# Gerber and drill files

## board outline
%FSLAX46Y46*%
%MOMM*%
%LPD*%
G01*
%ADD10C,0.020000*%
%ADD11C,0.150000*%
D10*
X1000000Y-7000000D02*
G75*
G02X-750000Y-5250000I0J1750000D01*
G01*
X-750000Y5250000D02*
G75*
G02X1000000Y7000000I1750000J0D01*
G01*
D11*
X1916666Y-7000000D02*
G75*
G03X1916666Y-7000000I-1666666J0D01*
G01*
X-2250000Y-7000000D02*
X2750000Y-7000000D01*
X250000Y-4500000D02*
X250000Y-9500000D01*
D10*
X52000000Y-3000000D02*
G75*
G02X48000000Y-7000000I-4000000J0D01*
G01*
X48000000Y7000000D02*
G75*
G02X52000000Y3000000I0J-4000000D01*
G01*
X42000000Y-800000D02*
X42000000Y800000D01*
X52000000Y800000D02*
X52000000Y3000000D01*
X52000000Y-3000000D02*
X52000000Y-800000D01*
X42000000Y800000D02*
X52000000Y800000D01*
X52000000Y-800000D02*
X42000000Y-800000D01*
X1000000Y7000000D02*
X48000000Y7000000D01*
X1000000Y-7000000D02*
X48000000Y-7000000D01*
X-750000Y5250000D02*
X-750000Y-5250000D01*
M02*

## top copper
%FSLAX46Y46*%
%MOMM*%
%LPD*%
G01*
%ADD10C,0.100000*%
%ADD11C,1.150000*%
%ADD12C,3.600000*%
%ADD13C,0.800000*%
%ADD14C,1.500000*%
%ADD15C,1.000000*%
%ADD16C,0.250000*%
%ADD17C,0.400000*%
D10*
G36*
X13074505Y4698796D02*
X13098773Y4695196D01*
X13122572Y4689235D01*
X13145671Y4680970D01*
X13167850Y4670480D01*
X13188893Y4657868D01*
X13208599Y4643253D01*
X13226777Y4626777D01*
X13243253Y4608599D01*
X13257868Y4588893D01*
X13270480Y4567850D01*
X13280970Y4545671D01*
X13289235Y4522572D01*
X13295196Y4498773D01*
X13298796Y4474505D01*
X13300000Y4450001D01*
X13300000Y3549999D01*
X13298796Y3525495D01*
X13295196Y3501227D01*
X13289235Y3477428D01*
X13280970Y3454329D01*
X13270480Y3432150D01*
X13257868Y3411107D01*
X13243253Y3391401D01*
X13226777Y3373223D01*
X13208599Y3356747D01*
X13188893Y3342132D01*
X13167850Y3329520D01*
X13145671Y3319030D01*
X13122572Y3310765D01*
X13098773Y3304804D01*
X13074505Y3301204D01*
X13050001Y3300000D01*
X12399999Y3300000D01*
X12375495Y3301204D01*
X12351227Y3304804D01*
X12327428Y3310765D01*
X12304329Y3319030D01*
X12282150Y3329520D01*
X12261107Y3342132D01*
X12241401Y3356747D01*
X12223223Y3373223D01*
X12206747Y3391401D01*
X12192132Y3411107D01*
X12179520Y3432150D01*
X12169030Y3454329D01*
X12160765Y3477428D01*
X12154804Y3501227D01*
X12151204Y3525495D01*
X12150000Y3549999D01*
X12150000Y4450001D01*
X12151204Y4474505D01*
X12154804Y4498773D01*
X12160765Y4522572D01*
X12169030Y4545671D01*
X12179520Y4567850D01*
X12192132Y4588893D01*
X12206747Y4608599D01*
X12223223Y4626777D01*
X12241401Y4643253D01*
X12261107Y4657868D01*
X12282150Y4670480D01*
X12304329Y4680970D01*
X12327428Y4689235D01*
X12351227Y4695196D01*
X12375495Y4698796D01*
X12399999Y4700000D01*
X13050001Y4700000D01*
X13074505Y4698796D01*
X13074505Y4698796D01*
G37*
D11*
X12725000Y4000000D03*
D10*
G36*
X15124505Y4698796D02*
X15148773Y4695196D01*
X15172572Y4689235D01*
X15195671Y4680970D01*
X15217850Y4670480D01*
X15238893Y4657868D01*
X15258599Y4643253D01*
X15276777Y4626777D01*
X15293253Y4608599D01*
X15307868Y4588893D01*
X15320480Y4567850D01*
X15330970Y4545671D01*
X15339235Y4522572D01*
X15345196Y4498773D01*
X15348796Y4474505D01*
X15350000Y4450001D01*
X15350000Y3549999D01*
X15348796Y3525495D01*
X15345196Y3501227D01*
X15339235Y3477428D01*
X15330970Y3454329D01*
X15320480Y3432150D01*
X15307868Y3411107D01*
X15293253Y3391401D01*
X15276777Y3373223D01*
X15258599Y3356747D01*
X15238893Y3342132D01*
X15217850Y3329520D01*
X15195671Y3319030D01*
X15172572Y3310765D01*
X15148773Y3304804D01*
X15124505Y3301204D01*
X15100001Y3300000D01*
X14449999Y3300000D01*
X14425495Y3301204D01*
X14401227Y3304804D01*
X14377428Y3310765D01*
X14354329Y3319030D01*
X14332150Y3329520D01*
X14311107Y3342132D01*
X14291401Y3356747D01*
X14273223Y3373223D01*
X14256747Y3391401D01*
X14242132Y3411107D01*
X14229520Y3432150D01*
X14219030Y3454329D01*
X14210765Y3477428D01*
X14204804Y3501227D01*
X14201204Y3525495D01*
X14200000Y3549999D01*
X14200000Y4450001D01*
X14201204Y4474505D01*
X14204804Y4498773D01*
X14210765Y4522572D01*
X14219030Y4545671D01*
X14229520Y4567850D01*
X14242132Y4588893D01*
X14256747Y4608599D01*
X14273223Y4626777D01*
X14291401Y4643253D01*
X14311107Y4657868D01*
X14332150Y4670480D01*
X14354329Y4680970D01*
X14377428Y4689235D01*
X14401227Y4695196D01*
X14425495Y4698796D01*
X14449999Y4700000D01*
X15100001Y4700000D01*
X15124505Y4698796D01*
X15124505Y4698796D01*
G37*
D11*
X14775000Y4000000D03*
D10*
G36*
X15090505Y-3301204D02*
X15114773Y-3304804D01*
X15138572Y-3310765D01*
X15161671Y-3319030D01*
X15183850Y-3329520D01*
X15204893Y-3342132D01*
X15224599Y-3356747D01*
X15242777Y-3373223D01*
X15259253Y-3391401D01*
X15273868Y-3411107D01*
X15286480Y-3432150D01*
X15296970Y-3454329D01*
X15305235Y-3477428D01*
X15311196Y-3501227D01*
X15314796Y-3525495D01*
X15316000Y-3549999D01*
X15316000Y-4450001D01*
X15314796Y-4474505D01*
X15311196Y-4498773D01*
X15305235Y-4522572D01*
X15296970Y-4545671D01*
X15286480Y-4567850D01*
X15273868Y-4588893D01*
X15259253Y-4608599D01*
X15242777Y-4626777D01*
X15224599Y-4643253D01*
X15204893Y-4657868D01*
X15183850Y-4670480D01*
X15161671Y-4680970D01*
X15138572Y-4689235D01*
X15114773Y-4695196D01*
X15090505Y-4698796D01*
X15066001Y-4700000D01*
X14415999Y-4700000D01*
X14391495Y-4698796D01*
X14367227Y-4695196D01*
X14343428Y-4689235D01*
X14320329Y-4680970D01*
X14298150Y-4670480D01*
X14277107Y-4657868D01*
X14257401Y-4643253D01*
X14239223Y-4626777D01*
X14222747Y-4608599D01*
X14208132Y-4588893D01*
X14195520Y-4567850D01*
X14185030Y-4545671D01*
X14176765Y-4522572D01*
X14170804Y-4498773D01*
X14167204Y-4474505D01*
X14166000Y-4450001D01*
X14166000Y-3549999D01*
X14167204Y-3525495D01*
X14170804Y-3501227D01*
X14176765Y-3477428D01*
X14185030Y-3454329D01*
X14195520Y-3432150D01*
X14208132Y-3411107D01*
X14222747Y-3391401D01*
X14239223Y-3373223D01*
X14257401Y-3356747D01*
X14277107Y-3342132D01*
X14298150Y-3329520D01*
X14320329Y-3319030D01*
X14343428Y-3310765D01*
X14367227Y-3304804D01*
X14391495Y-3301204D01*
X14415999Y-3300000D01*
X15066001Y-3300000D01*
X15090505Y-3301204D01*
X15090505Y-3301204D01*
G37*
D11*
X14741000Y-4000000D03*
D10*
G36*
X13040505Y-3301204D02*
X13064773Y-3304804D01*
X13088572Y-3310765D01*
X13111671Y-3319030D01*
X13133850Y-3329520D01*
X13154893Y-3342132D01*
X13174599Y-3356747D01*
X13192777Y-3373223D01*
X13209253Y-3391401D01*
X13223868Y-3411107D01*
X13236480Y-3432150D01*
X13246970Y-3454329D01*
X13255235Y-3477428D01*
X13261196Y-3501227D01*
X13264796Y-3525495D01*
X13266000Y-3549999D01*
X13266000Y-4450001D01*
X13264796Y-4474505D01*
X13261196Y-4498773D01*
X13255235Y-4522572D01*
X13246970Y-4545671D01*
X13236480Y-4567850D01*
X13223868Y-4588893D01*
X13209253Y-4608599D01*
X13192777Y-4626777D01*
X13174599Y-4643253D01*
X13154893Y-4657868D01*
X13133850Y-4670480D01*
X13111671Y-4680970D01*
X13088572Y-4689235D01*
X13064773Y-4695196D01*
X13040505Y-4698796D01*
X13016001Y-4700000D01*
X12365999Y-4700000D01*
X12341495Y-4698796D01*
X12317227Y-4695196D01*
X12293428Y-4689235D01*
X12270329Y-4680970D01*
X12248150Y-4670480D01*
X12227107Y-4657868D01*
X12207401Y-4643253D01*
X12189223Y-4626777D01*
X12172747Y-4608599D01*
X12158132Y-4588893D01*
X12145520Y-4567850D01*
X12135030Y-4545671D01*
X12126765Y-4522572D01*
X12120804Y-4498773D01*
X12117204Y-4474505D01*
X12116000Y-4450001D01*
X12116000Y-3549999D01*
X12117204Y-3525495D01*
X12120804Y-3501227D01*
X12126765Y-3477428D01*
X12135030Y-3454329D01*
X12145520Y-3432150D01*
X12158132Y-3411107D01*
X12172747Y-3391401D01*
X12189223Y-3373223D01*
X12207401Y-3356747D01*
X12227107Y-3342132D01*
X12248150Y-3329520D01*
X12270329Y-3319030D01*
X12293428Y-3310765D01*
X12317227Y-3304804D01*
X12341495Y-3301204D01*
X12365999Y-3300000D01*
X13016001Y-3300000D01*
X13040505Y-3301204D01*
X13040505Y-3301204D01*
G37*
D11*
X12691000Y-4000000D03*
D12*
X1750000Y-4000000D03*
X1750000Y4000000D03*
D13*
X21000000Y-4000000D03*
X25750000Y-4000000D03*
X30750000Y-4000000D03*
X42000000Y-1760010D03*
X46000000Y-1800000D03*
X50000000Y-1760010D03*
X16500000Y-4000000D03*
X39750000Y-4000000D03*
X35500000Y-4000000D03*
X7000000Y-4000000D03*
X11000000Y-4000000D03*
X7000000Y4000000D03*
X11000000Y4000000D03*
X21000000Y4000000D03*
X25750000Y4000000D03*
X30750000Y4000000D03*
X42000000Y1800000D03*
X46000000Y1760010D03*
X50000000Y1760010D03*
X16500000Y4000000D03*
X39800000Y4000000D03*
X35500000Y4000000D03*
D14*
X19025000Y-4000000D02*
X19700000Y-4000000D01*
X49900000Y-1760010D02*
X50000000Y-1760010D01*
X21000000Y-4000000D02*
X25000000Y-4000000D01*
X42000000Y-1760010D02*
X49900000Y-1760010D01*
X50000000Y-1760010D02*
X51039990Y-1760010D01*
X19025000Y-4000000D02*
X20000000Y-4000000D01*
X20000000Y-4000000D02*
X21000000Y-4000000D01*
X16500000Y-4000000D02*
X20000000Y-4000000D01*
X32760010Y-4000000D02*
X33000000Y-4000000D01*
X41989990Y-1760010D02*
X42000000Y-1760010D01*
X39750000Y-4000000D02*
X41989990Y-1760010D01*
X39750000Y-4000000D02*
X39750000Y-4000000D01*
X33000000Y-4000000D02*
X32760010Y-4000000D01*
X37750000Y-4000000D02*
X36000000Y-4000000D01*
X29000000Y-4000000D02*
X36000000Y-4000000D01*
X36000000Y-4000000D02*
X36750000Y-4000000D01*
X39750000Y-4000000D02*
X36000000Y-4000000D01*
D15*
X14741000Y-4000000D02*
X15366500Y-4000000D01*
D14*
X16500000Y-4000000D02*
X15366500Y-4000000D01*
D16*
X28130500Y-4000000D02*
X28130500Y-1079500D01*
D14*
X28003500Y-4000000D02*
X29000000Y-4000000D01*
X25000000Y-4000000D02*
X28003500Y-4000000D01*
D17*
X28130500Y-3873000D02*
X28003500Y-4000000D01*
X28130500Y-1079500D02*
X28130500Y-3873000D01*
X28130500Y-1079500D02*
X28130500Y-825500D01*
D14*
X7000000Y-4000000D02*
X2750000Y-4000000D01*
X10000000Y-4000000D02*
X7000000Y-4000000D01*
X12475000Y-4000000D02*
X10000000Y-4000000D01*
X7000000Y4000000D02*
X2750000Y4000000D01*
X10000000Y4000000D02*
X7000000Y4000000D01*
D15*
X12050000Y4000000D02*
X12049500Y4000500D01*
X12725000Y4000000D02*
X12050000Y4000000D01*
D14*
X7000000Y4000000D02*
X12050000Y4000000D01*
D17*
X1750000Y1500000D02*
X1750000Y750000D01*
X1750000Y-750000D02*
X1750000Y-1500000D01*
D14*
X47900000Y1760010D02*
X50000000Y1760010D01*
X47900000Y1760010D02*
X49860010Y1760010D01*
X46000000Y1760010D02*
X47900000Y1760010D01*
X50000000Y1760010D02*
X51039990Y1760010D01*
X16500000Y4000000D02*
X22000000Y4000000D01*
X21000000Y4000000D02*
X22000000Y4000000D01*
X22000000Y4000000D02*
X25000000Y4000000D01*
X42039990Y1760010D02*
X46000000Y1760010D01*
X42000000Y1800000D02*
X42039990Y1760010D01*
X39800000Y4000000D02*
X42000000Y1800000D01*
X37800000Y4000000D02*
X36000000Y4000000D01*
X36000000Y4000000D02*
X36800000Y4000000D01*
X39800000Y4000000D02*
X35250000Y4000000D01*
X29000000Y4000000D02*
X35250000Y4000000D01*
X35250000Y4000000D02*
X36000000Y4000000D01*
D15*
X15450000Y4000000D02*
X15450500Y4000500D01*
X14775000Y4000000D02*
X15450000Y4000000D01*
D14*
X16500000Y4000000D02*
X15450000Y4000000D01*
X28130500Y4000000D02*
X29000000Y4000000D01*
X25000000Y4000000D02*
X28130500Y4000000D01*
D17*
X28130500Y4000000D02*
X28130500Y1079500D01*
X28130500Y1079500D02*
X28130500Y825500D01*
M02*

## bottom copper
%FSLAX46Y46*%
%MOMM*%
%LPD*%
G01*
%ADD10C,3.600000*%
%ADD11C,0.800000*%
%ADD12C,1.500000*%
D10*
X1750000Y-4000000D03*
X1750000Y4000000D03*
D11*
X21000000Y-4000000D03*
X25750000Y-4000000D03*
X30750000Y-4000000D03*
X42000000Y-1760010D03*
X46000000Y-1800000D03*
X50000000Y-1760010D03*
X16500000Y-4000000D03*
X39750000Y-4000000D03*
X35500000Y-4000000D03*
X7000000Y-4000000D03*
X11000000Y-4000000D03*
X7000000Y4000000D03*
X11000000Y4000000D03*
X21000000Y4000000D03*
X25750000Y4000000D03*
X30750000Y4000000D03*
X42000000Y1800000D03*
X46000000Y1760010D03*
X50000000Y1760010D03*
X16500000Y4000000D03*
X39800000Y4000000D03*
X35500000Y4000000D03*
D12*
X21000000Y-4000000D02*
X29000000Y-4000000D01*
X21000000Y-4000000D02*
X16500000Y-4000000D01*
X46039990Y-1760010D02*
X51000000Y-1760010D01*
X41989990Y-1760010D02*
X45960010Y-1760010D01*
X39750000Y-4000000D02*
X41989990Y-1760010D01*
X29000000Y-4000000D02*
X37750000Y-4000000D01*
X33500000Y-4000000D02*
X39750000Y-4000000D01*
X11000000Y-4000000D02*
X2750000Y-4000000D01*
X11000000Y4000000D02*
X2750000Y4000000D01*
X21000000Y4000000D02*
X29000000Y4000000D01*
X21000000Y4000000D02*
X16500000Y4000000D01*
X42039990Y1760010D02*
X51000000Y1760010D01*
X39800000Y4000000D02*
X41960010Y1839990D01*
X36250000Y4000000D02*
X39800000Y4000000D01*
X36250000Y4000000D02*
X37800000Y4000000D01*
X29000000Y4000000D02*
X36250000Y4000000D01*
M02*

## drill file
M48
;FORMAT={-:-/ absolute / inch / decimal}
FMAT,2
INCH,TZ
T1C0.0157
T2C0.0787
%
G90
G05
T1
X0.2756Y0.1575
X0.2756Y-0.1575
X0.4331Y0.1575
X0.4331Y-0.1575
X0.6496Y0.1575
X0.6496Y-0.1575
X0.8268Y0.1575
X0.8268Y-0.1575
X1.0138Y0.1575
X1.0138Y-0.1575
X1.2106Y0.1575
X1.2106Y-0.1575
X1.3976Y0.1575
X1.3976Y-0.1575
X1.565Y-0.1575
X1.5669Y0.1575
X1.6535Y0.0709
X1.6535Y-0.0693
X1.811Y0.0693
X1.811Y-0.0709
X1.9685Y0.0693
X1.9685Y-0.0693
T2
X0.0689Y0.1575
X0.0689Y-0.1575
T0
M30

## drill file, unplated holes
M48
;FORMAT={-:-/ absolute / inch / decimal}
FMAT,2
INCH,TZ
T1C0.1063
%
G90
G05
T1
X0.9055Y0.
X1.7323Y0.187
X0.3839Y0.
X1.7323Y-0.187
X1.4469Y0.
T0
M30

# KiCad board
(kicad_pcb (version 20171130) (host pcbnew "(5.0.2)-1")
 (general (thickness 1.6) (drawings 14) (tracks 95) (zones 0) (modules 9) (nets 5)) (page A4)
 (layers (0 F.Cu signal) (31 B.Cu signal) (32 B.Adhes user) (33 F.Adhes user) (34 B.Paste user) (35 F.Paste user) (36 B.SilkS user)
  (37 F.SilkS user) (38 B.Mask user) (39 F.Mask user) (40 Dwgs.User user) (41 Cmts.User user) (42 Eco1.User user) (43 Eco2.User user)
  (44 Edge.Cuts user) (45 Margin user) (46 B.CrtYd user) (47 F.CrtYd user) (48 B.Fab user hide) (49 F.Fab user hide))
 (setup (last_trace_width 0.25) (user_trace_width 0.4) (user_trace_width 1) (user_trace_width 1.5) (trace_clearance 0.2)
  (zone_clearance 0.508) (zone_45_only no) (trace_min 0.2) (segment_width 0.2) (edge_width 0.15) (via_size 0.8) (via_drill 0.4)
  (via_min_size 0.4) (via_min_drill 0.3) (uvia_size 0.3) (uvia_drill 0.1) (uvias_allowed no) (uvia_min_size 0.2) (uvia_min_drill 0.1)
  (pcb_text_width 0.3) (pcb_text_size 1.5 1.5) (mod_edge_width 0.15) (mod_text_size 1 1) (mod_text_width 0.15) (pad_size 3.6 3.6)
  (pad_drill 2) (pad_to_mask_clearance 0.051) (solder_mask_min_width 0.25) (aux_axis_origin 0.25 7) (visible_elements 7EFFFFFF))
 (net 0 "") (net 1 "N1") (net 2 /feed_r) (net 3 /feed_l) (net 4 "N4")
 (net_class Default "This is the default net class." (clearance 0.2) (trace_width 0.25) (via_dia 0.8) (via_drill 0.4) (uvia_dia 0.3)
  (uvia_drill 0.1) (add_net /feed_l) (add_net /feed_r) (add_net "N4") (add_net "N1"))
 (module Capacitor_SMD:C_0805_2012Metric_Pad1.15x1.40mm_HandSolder (layer F.Cu) (at 13.75 -4 180)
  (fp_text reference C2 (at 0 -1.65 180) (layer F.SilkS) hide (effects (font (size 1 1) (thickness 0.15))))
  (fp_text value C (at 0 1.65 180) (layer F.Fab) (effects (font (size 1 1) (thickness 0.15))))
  (pad 2 smd roundrect (at 1.025 0 180) (size 1.15 1.4) (layers F.Cu F.Paste F.Mask) (roundrect_rratio 0.217391) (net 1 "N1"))
  (pad 1 smd roundrect (at -1.025 0 180) (size 1.15 1.4) (layers F.Cu F.Paste F.Mask) (roundrect_rratio 0.217391) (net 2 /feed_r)))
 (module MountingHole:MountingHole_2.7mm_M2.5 (layer F.Cu) (at 23 0)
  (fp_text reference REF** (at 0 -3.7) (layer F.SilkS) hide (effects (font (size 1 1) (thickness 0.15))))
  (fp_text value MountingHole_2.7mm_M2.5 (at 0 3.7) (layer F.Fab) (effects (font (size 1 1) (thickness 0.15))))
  (pad 1 np_thru_hole circle (at 0 0) (size 2.7 2.7) (drill 2.7) (layers *.Cu *.Mask)))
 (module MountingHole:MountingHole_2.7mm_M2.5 (layer F.Cu) (at 44 -4.75)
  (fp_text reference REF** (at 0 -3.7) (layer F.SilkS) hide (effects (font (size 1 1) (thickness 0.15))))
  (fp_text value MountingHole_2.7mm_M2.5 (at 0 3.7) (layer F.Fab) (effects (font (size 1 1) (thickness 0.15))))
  (pad 1 np_thru_hole circle (at 0 0) (size 2.7 2.7) (drill 2.7) (layers *.Cu *.Mask)))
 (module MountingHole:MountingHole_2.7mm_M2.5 (layer F.Cu) (at 44 4.75)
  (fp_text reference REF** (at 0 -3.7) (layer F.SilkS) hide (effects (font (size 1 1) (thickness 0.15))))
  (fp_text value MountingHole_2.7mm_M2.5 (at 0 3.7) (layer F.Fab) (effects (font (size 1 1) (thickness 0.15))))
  (pad 1 np_thru_hole circle (at 0 0) (size 2.7 2.7) (drill 2.7) (layers *.Cu *.Mask)))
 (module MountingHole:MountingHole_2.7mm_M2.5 (layer F.Cu) (at 36.75 0)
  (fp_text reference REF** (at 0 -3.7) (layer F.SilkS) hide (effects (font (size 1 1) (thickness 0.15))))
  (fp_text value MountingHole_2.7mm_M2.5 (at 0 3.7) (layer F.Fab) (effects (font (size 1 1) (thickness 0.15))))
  (pad 1 np_thru_hole circle (at 0 0) (size 2.7 2.7) (drill 2.7) (layers *.Cu *.Mask)))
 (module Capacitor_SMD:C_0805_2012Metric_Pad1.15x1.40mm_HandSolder (layer F.Cu) (at 13.716 4 180)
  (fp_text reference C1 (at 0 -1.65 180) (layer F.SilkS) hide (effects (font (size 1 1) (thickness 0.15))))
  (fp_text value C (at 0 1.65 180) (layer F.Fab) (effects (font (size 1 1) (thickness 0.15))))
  (pad 1 smd roundrect (at -1.025 0 180) (size 1.15 1.4) (layers F.Cu F.Paste F.Mask) (roundrect_rratio 0.217391) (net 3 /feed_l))
  (pad 2 smd roundrect (at 1.025 0 180) (size 1.15 1.4) (layers F.Cu F.Paste F.Mask) (roundrect_rratio 0.217391) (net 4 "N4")))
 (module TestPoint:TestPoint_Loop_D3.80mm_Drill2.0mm (layer F.Cu) (at 1.75 4)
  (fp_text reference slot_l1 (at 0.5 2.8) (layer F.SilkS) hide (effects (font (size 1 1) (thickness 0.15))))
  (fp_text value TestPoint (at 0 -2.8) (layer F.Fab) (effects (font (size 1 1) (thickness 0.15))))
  (pad 1 thru_hole circle (at 0 0) (size 3.6 3.6) (drill 2) (layers *.Cu *.Mask) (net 4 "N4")))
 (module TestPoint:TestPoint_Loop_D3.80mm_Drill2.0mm (layer F.Cu) (at 1.75 -4)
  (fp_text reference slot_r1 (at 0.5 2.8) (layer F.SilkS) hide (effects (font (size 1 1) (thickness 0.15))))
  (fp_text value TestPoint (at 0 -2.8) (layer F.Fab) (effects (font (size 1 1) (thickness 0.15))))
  (pad 1 thru_hole circle (at 0 0) (size 3.6 3.6) (drill 2) (layers *.Cu *.Mask) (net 1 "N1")))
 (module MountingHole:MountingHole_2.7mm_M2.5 (layer F.Cu) (at 9.75 0)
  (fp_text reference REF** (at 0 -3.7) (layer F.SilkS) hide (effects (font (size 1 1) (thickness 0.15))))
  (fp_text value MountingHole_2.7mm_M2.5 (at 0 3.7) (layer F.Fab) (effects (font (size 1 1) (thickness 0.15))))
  (pad 1 np_thru_hole circle (at 0 0) (size 2.7 2.7) (drill 2.7) (layers *.Cu *.Mask)))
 (gr_arc (start 1 5.25) (end -0.75 5.25) (angle -90) (layer Edge.Cuts) (width 0.02))
 (gr_arc (start 1 -5.25) (end 1 -7) (angle -90) (layer Edge.Cuts) (width 0.02))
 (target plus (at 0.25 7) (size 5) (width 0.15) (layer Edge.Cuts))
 (gr_arc (start 48 3) (end 48 7) (angle -90) (layer Edge.Cuts) (width 0.02))
 (gr_arc (start 48 -3) (end 52 -3) (angle -90) (layer Edge.Cuts) (width 0.02))
 (gr_line (start 42 0.8) (end 42 -0.8) (layer Edge.Cuts) (width 0.02))
 (gr_line (start 52 -0.8) (end 52 -3) (layer Edge.Cuts) (width 0.02))
 (gr_line (start 52 3) (end 52 0.8) (layer Edge.Cuts) (width 0.02))
 (gr_line (start 42 -0.8) (end 52 -0.8) (layer Edge.Cuts) (width 0.02))
 (gr_line (start 52 0.8) (end 42 0.8) (layer Edge.Cuts) (width 0.02))
 (gr_line (start 1 -7) (end 48 -7) (layer Edge.Cuts) (width 0.02))
 (gr_line (start 1 7) (end 48 7) (layer Edge.Cuts) (width 0.02))
 (gr_line (start -0.75 -5.25) (end -0.75 5.25) (layer Edge.Cuts) (width 0.02))
 (segment (start 19.025 4) (end 19.7 4) (width 1.5) (layer F.Cu) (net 3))
 (segment (start 49.9 1.76001) (end 50 1.76001) (width 1.5) (layer F.Cu) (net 3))
 (segment (start 21 4) (end 25 4) (width 1.5) (layer F.Cu) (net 3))
 (via (at 21 4) (size 0.8) (drill 0.4) (layers F.Cu B.Cu) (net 3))
 (segment (start 21 4) (end 29 4) (width 1.5) (layer B.Cu) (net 3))
 (via (at 25.75 4) (size 0.8) (drill 0.4) (layers F.Cu B.Cu) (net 3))
 (via (at 30.75 4) (size 0.8) (drill 0.4) (layers F.Cu B.Cu) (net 3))
 (segment (start 42 1.76001) (end 49.9 1.76001) (width 1.5) (layer F.Cu) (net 3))
 (via (at 42 1.76001) (size 0.8) (drill 0.4) (layers F.Cu B.Cu) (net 3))
 (via (at 46 1.8) (size 0.8) (drill 0.4) (layers F.Cu B.Cu) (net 3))
 (via (at 50 1.76001) (size 0.8) (drill 0.4) (layers F.Cu B.Cu) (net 3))
 (segment (start 50 1.76001) (end 51.03999 1.76001) (width 1.5) (layer F.Cu) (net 3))
 (segment (start 19.025 4) (end 20 4) (width 1.5) (layer F.Cu) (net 3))
 (segment (start 20 4) (end 21 4) (width 1.5) (layer F.Cu) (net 3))
 (segment (start 16.5 4) (end 20 4) (width 1.5) (layer F.Cu) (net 3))
 (via (at 16.5 4) (size 0.8) (drill 0.4) (layers F.Cu B.Cu) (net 3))
 (segment (start 21 4) (end 16.5 4) (width 1.5) (layer B.Cu) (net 3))
 (segment (start 32.76001 4) (end 33 4) (width 1.5) (layer F.Cu) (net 3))
 (segment (start 46.03999 1.76001) (end 51 1.76001) (width 1.5) (layer B.Cu) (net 3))
 (segment (start 41.98999 1.76001) (end 42 1.76001) (width 1.5) (layer F.Cu) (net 3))
 (segment (start 39.75 4) (end 41.98999 1.76001) (width 1.5) (layer F.Cu) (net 3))
 (segment (start 41.98999 1.76001) (end 45.96001 1.76001) (width 1.5) (layer B.Cu) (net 3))
 (segment (start 39.75 4) (end 41.98999 1.76001) (width 1.5) (layer B.Cu) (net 3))
 (segment (start 39.75 4) (end 39.75 4) (width 1.5) (layer F.Cu) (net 3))
 (via (at 39.75 4) (size 0.8) (drill 0.4) (layers F.Cu B.Cu) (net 3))
 (segment (start 33 4) (end 32.76001 4) (width 1.5) (layer F.Cu) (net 3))
 (via (at 35.5 4) (size 0.8) (drill 0.4) (layers F.Cu B.Cu) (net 3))
 (segment (start 37.75 4) (end 36 4) (width 1.5) (layer F.Cu) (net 3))
 (segment (start 29 4) (end 36 4) (width 1.5) (layer F.Cu) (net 3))
 (segment (start 36 4) (end 36.75 4) (width 1.5) (layer F.Cu) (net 3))
 (segment (start 29 4) (end 37.75 4) (width 1.5) (layer B.Cu) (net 3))
 (segment (start 39.75 4) (end 36 4) (width 1.5) (layer F.Cu) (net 3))
 (segment (start 33.5 4) (end 39.75 4) (width 1.5) (layer B.Cu) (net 3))
 (segment (start 14.741 4) (end 15.3665 4) (width 1) (layer F.Cu) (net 3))
 (segment (start 16.5 4) (end 15.3665 4) (width 1.5) (layer F.Cu) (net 3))
 (segment (start 28.1305 4) (end 28.1305 1.0795) (width 0.25) (layer F.Cu) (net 3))
 (segment (start 28.0035 4) (end 29 4) (width 1.5) (layer F.Cu) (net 3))
 (segment (start 25 4) (end 28.0035 4) (width 1.5) (layer F.Cu) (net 3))
 (segment (start 28.1305 3.873) (end 28.0035 4) (width 0.4) (layer F.Cu) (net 3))
 (segment (start 28.1305 1.0795) (end 28.1305 3.873) (width 0.4) (layer F.Cu) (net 3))
 (segment (start 28.1305 1.0795) (end 28.1305 0.8255) (width 0.4) (layer F.Cu) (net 3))
 (segment (start 7 4) (end 2.75 4) (width 1.5) (layer F.Cu) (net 4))
 (via (at 7 4) (size 0.8) (drill 0.4) (layers F.Cu B.Cu) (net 4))
 (segment (start 10 4) (end 7 4) (width 1.5) (layer F.Cu) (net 4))
 (via (at 11 4) (size 0.8) (drill 0.4) (layers F.Cu B.Cu) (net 4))
 (segment (start 11 4) (end 2.75 4) (width 1.5) (layer B.Cu) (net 4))
 (segment (start 12.475 4) (end 10 4) (width 1.5) (layer F.Cu) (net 4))
 (segment (start 7 -4) (end 2.75 -4) (width 1.5) (layer F.Cu) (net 1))
 (via (at 7 -4) (size 0.8) (drill 0.4) (layers F.Cu B.Cu) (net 1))
 (segment (start 10 -4) (end 7 -4) (width 1.5) (layer F.Cu) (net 1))
 (via (at 11 -4) (size 0.8) (drill 0.4) (layers F.Cu B.Cu) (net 1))
 (segment (start 11 -4) (end 2.75 -4) (width 1.5) (layer B.Cu) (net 1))
 (segment (start 12.05 -4) (end 12.0495 -4.0005) (width 1) (layer F.Cu) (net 1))
 (segment (start 12.725 -4) (end 12.05 -4) (width 1) (layer F.Cu) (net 1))
 (segment (start 7 -4) (end 12.05 -4) (width 1.5) (layer F.Cu) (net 1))
 (segment (start 1.75 -1.5) (end 1.75 -0.75) (width 0.4) (layer F.Cu) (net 1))
 (segment (start 1.75 0.75) (end 1.75 1.5) (width 0.4) (layer F.Cu) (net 1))
 (segment (start 47.9 -1.76001) (end 50 -1.76001) (width 1.5) (layer F.Cu) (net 2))
 (segment (start 47.9 -1.76001) (end 49.86001 -1.76001) (width 1.5) (layer F.Cu) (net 2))
 (via (at 21 -4) (size 0.8) (drill 0.4) (layers F.Cu B.Cu) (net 2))
 (segment (start 21 -4) (end 29 -4) (width 1.5) (layer B.Cu) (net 2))
 (via (at 25.75 -4) (size 0.8) (drill 0.4) (layers F.Cu B.Cu) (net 2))
 (via (at 30.75 -4) (size 0.8) (drill 0.4) (layers F.Cu B.Cu) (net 2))
 (via (at 42 -1.8) (size 0.8) (drill 0.4) (layers F.Cu B.Cu) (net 2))
 (segment (start 46 -1.76001) (end 47.9 -1.76001) (width 1.5) (layer F.Cu) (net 2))
 (via (at 46 -1.76001) (size 0.8) (drill 0.4) (layers F.Cu B.Cu) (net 2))
 (via (at 50 -1.76001) (size 0.8) (drill 0.4) (layers F.Cu B.Cu) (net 2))
 (segment (start 50 -1.76001) (end 51.03999 -1.76001) (width 1.5) (layer F.Cu) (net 2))
 (via (at 16.5 -4) (size 0.8) (drill 0.4) (layers F.Cu B.Cu) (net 2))
 (segment (start 21 -4) (end 16.5 -4) (width 1.5) (layer B.Cu) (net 2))
 (segment (start 42.03999 -1.76001) (end 51 -1.76001) (width 1.5) (layer B.Cu) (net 2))
 (segment (start 16.5 -4) (end 22 -4) (width 1.5) (layer F.Cu) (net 2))
 (segment (start 21 -4) (end 22 -4) (width 1.5) (layer F.Cu) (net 2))
 (segment (start 22 -4) (end 25 -4) (width 1.5) (layer F.Cu) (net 2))
 (segment (start 42.03999 -1.76001) (end 46 -1.76001) (width 1.5) (layer F.Cu) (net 2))
 (segment (start 42 -1.8) (end 42.03999 -1.76001) (width 1.5) (layer F.Cu) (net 2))
 (segment (start 39.8 -4) (end 41.96001 -1.83999) (width 1.5) (layer B.Cu) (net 2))
 (segment (start 39.8 -4) (end 42 -1.8) (width 1.5) (layer F.Cu) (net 2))
 (via (at 39.8 -4) (size 0.8) (drill 0.4) (layers F.Cu B.Cu) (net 2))
 (via (at 35.5 -4) (size 0.8) (drill 0.4) (layers F.Cu B.Cu) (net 2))
 (segment (start 37.8 -4) (end 36 -4) (width 1.5) (layer F.Cu) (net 2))
 (segment (start 36 -4) (end 36.8 -4) (width 1.5) (layer F.Cu) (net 2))
 (segment (start 39.8 -4) (end 35.25 -4) (width 1.5) (layer F.Cu) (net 2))
 (segment (start 29 -4) (end 35.25 -4) (width 1.5) (layer F.Cu) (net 2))
 (segment (start 35.25 -4) (end 36 -4) (width 1.5) (layer F.Cu) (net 2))
 (segment (start 36.25 -4) (end 39.8 -4) (width 1.5) (layer B.Cu) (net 2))
 (segment (start 36.25 -4) (end 37.8 -4) (width 1.5) (layer B.Cu) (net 2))
 (segment (start 29 -4) (end 36.25 -4) (width 1.5) (layer B.Cu) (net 2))
 (segment (start 15.45 -4) (end 15.4505 -4.0005) (width 1) (layer F.Cu) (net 2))
 (segment (start 14.775 -4) (end 15.45 -4) (width 1) (layer F.Cu) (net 2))
 (segment (start 16.5 -4) (end 15.45 -4) (width 1.5) (layer F.Cu) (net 2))
 (segment (start 28.1305 -4) (end 29 -4) (width 1.5) (layer F.Cu) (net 2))
 (segment (start 25 -4) (end 28.1305 -4) (width 1.5) (layer F.Cu) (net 2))
 (segment (start 28.1305 -4) (end 28.1305 -1.0795) (width 0.4) (layer F.Cu) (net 2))
 (segment (start 28.1305 -1.0795) (end 28.1305 -0.8255) (width 0.4) (layer F.Cu) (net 2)))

